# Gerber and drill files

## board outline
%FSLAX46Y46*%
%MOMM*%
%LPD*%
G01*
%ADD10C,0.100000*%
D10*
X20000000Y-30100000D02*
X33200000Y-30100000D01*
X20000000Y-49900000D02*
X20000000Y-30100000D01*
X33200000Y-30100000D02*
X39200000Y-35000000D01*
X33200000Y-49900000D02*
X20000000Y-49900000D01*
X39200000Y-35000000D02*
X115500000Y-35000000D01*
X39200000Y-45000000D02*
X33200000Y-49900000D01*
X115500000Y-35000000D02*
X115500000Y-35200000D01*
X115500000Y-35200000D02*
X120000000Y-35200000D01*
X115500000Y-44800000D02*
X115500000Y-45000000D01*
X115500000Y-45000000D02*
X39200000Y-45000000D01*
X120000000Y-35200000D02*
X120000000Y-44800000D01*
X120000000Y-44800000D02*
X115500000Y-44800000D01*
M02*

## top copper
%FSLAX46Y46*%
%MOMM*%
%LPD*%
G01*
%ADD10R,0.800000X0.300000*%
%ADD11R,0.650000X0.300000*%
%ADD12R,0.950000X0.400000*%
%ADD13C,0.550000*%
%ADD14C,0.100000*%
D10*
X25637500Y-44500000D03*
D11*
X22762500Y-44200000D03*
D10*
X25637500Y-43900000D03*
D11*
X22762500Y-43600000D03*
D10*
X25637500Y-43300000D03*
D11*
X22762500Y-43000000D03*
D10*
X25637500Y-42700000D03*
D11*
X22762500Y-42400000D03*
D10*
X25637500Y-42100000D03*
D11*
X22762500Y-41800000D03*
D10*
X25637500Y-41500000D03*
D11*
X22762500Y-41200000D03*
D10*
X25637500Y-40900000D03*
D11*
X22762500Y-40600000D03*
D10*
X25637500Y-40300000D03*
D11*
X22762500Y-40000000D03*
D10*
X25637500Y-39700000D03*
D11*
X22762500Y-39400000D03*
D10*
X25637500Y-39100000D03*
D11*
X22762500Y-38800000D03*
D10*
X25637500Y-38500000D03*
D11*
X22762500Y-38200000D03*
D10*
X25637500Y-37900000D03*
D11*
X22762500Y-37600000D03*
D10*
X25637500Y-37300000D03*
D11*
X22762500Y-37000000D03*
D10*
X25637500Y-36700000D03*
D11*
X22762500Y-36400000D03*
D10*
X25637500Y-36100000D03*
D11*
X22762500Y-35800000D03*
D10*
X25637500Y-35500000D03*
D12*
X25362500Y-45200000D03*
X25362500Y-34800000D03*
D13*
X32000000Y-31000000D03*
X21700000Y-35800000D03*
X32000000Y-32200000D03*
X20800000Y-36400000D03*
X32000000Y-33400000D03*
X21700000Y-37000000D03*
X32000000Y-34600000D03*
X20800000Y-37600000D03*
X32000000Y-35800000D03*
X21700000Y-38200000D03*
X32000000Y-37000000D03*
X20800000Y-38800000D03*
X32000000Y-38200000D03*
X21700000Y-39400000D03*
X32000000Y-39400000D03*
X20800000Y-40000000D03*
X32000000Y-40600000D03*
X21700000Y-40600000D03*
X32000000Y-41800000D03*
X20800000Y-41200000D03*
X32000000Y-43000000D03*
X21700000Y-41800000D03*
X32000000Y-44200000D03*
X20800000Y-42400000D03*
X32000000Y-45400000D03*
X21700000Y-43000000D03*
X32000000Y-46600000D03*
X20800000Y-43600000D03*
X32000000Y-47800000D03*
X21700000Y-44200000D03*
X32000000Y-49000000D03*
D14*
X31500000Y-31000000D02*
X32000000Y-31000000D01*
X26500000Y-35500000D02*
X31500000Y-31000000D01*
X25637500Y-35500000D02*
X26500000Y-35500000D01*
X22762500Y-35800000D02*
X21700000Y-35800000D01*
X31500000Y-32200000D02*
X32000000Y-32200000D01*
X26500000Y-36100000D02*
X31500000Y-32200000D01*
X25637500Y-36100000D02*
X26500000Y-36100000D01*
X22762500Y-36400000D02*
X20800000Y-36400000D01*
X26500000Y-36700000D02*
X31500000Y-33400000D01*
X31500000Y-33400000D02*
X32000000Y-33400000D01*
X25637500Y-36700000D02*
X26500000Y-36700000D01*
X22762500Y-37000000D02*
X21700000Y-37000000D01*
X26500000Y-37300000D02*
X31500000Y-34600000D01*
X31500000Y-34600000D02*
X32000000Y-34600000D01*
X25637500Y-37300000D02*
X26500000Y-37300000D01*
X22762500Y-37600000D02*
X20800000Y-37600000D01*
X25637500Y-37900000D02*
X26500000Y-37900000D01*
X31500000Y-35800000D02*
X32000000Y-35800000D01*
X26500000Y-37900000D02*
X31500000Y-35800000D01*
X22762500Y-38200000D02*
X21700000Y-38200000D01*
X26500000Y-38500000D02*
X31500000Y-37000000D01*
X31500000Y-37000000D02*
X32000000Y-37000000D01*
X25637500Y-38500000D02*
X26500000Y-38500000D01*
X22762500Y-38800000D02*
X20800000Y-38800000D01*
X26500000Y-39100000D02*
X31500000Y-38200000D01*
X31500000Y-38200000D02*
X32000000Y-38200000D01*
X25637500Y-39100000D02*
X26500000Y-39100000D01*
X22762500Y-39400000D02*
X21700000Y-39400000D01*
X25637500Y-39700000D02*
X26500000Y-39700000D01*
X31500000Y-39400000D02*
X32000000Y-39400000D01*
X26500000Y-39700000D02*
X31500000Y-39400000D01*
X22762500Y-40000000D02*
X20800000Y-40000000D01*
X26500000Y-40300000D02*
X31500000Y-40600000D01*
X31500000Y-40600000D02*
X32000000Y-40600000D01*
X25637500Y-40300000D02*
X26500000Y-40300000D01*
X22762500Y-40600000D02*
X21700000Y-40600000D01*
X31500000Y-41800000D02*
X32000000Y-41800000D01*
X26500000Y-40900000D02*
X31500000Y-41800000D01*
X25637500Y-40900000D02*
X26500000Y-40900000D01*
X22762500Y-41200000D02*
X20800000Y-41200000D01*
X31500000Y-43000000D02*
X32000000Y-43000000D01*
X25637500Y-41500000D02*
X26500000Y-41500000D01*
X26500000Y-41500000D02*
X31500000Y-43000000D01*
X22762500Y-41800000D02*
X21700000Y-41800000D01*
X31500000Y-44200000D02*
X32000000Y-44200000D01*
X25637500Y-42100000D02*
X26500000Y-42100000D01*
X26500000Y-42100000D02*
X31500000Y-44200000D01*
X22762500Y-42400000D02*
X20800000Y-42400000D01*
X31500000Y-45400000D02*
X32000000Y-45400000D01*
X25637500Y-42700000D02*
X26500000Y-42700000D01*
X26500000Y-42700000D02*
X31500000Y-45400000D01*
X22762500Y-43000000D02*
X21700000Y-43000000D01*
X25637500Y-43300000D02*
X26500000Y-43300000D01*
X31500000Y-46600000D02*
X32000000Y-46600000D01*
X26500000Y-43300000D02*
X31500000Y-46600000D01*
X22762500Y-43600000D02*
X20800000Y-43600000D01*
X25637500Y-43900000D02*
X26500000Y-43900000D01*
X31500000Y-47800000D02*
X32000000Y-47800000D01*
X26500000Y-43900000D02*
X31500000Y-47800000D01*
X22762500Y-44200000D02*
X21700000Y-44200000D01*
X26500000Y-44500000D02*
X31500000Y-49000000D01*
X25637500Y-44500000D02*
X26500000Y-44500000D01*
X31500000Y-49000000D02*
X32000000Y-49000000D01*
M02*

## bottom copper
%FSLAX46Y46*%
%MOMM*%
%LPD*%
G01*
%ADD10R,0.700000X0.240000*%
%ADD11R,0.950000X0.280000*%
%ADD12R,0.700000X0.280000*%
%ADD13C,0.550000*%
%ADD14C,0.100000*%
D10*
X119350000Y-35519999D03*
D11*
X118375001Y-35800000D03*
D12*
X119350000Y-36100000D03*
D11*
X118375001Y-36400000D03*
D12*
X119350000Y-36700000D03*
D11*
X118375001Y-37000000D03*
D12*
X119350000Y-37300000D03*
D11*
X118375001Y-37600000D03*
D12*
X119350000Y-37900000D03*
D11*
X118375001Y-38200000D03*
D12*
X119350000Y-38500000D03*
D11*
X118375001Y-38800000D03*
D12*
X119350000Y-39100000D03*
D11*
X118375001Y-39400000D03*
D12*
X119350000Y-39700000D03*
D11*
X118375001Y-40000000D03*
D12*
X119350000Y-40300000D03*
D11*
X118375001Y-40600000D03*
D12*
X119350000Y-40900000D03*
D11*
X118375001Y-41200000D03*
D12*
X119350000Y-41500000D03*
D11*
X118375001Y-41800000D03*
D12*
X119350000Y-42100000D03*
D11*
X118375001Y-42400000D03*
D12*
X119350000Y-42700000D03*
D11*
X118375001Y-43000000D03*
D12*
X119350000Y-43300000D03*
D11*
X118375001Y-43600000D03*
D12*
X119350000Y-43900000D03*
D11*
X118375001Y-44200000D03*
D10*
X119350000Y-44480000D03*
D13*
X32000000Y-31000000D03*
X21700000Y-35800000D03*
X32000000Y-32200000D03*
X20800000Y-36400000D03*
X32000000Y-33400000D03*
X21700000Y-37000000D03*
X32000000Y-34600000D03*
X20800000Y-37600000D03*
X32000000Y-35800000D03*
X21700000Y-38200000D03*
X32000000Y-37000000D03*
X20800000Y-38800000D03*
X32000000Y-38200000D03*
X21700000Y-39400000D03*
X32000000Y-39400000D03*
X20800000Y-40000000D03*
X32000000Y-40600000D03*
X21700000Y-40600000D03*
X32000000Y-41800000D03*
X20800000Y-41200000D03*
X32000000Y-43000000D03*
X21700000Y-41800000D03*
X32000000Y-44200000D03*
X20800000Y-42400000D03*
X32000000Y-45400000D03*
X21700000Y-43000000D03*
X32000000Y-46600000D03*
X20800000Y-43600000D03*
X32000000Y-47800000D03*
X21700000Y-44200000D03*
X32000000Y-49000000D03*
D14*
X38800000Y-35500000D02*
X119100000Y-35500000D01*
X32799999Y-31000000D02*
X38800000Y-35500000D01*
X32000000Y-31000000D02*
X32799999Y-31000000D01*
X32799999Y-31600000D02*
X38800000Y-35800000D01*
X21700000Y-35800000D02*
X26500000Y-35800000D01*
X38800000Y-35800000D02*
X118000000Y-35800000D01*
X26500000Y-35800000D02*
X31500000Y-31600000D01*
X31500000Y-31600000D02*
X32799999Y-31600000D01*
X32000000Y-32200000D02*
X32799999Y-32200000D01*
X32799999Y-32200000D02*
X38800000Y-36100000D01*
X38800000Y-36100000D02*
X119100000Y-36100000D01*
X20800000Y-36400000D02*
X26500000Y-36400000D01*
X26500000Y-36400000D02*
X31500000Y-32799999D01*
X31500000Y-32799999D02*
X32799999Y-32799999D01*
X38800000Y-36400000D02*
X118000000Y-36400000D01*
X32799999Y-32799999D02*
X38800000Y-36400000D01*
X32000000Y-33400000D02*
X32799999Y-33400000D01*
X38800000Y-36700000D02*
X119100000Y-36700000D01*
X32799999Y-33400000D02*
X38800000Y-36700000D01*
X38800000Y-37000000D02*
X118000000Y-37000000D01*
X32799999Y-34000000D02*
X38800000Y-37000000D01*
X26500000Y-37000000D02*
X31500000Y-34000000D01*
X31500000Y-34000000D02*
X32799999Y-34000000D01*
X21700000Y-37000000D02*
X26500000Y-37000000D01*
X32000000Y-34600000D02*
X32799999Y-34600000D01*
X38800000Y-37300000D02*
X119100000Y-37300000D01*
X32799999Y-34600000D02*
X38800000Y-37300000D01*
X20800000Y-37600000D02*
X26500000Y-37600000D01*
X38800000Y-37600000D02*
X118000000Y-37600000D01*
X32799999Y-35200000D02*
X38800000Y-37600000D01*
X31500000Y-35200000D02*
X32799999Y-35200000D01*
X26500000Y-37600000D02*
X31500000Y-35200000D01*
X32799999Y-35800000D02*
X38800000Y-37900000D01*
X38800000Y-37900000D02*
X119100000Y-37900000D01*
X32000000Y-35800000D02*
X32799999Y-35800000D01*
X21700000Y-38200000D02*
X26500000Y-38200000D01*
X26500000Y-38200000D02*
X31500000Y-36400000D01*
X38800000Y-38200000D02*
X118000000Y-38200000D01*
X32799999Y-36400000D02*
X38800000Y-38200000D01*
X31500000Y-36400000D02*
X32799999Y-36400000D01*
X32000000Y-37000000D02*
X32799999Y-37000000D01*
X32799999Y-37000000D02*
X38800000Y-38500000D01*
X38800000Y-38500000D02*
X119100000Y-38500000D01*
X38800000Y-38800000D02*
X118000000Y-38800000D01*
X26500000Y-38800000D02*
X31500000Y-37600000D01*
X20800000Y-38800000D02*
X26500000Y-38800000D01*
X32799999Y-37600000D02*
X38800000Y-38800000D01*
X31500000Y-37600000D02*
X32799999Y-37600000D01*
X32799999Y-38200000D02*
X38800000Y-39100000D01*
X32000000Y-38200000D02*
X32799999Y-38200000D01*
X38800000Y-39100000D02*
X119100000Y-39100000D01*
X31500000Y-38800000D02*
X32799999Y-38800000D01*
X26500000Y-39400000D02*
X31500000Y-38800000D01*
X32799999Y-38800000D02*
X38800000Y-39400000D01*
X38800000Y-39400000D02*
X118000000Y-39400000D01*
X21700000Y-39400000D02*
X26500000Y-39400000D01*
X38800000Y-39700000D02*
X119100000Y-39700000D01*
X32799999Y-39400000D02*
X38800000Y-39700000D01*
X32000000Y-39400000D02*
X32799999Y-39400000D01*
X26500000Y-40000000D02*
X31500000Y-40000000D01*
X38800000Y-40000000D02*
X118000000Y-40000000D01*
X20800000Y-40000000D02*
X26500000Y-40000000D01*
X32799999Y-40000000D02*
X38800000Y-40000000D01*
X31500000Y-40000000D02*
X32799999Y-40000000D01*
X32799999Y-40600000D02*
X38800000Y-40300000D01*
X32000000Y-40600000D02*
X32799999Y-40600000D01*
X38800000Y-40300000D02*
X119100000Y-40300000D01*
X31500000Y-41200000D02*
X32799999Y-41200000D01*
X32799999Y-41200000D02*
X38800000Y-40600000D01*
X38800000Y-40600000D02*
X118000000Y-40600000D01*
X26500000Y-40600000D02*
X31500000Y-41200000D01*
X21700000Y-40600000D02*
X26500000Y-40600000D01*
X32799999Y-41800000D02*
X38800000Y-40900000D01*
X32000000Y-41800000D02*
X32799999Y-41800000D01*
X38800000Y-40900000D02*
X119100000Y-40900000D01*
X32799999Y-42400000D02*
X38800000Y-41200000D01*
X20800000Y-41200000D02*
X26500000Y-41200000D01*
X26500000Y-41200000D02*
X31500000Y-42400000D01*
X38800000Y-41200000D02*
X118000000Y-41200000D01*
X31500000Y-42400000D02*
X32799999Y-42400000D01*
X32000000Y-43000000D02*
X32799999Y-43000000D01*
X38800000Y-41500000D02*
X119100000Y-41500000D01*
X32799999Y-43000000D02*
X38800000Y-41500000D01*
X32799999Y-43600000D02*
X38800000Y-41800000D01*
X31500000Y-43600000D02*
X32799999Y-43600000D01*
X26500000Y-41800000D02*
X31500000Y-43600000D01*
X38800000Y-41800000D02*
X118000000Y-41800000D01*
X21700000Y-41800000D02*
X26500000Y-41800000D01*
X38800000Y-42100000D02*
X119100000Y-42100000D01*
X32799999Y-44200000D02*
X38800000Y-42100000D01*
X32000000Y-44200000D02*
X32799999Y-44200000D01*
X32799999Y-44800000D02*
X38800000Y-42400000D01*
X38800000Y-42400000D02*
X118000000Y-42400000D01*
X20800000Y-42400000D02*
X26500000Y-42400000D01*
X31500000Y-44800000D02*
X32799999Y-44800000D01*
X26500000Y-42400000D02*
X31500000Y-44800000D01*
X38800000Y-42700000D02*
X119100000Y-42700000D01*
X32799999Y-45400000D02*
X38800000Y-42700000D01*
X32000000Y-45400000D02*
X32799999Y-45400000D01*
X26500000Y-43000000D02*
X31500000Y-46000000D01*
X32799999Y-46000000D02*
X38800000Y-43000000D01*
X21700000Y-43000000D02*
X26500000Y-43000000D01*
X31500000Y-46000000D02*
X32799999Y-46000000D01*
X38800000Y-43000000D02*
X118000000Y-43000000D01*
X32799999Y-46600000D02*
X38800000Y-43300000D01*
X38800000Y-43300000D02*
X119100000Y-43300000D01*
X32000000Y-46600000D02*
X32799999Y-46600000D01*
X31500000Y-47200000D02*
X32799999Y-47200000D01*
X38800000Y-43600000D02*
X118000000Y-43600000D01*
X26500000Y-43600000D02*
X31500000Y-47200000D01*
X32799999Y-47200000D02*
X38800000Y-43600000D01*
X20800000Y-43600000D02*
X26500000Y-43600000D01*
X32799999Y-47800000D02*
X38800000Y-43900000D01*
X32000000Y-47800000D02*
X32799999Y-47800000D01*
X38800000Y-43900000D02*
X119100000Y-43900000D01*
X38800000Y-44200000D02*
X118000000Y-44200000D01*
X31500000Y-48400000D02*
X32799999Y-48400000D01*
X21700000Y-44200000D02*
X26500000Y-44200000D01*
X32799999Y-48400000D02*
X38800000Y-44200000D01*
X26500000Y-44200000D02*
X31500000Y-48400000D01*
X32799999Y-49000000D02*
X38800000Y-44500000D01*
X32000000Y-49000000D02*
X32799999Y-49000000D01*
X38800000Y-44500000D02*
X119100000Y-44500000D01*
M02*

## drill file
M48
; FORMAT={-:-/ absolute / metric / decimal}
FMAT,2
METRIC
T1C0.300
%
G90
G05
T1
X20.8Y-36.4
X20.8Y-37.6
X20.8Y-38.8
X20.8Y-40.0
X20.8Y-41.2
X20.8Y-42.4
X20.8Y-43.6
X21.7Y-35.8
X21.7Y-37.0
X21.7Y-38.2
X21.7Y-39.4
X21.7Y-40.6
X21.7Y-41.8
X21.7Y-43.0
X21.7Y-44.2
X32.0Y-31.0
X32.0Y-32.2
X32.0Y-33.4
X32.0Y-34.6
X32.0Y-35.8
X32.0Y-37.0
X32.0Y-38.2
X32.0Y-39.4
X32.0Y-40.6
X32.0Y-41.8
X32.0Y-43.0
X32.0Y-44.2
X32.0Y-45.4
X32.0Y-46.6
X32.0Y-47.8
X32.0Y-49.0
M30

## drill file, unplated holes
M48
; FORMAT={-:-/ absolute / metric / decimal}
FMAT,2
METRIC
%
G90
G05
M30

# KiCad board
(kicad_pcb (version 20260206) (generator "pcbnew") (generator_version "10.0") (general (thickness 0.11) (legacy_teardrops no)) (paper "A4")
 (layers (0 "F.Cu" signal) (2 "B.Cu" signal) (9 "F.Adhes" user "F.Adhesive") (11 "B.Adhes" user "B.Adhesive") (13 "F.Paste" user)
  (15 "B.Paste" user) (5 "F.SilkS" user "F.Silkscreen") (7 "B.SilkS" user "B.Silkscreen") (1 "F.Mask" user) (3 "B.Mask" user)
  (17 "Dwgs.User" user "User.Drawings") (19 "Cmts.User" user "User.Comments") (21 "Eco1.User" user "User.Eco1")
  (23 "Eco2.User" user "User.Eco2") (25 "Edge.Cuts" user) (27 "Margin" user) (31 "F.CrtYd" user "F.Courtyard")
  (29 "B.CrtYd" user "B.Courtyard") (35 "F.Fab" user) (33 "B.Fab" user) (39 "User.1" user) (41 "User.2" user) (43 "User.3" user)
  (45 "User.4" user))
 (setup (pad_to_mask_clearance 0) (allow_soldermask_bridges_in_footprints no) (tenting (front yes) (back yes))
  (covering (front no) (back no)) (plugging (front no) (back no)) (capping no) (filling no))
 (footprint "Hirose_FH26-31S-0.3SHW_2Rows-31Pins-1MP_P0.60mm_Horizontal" (layer "F.Cu") (at 24.2375 40 180)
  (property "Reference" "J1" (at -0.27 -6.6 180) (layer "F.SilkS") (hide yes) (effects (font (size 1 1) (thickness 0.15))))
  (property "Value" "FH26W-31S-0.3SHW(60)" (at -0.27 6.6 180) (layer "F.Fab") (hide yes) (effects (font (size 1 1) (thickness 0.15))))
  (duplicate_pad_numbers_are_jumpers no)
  (pad "1" smd rect (at -1.4 -4.5 180) (size 0.8 0.3) (layers "F.Cu" "F.Mask" "F.Paste") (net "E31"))
  (pad "2" smd rect (at 1.475 -4.2 180) (size 0.65 0.3) (layers "F.Cu" "F.Mask" "F.Paste") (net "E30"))
  (pad "3" smd rect (at -1.4 -3.9 180) (size 0.8 0.3) (layers "F.Cu" "F.Mask" "F.Paste") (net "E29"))
  (pad "4" smd rect (at 1.475 -3.6 180) (size 0.65 0.3) (layers "F.Cu" "F.Mask" "F.Paste") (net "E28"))
  (pad "5" smd rect (at -1.4 -3.3 180) (size 0.8 0.3) (layers "F.Cu" "F.Mask" "F.Paste") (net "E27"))
  (pad "6" smd rect (at 1.475 -3 180) (size 0.65 0.3) (layers "F.Cu" "F.Mask" "F.Paste") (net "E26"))
  (pad "7" smd rect (at -1.4 -2.7 180) (size 0.8 0.3) (layers "F.Cu" "F.Mask" "F.Paste") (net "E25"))
  (pad "8" smd rect (at 1.475 -2.4 180) (size 0.65 0.3) (layers "F.Cu" "F.Mask" "F.Paste") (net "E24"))
  (pad "9" smd rect (at -1.4 -2.1 180) (size 0.8 0.3) (layers "F.Cu" "F.Mask" "F.Paste") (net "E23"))
  (pad "10" smd rect (at 1.475 -1.8 180) (size 0.65 0.3) (layers "F.Cu" "F.Mask" "F.Paste") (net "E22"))
  (pad "11" smd rect (at -1.4 -1.5 180) (size 0.8 0.3) (layers "F.Cu" "F.Mask" "F.Paste") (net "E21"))
  (pad "12" smd rect (at 1.475 -1.2 180) (size 0.65 0.3) (layers "F.Cu" "F.Mask" "F.Paste") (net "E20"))
  (pad "13" smd rect (at -1.4 -0.9 180) (size 0.8 0.3) (layers "F.Cu" "F.Mask" "F.Paste") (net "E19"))
  (pad "14" smd rect (at 1.475 -0.6 180) (size 0.65 0.3) (layers "F.Cu" "F.Mask" "F.Paste") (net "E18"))
  (pad "15" smd rect (at -1.4 -0.3 180) (size 0.8 0.3) (layers "F.Cu" "F.Mask" "F.Paste") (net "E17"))
  (pad "16" smd rect (at 1.475 0 180) (size 0.65 0.3) (layers "F.Cu" "F.Mask" "F.Paste") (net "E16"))
  (pad "17" smd rect (at -1.4 0.3 180) (size 0.8 0.3) (layers "F.Cu" "F.Mask" "F.Paste") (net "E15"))
  (pad "18" smd rect (at 1.475 0.6 180) (size 0.65 0.3) (layers "F.Cu" "F.Mask" "F.Paste") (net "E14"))
  (pad "19" smd rect (at -1.4 0.9 180) (size 0.8 0.3) (layers "F.Cu" "F.Mask" "F.Paste") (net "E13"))
  (pad "20" smd rect (at 1.475 1.2 180) (size 0.65 0.3) (layers "F.Cu" "F.Mask" "F.Paste") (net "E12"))
  (pad "21" smd rect (at -1.4 1.5 180) (size 0.8 0.3) (layers "F.Cu" "F.Mask" "F.Paste") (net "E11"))
  (pad "22" smd rect (at 1.475 1.8 180) (size 0.65 0.3) (layers "F.Cu" "F.Mask" "F.Paste") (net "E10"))
  (pad "23" smd rect (at -1.4 2.1 180) (size 0.8 0.3) (layers "F.Cu" "F.Mask" "F.Paste") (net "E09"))
  (pad "24" smd rect (at 1.475 2.4 180) (size 0.65 0.3) (layers "F.Cu" "F.Mask" "F.Paste") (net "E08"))
  (pad "25" smd rect (at -1.4 2.7 180) (size 0.8 0.3) (layers "F.Cu" "F.Mask" "F.Paste") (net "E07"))
  (pad "26" smd rect (at 1.475 3 180) (size 0.65 0.3) (layers "F.Cu" "F.Mask" "F.Paste") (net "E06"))
  (pad "27" smd rect (at -1.4 3.3 180) (size 0.8 0.3) (layers "F.Cu" "F.Mask" "F.Paste") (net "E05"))
  (pad "28" smd rect (at 1.475 3.6 180) (size 0.65 0.3) (layers "F.Cu" "F.Mask" "F.Paste") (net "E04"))
  (pad "29" smd rect (at -1.4 3.9 180) (size 0.8 0.3) (layers "F.Cu" "F.Mask" "F.Paste") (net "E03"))
  (pad "30" smd rect (at 1.475 4.2 180) (size 0.65 0.3) (layers "F.Cu" "F.Mask" "F.Paste") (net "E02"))
  (pad "31" smd rect (at -1.4 4.5 180) (size 0.8 0.3) (layers "F.Cu" "F.Mask" "F.Paste") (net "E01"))
  (pad "MP" smd rect (at -1.125 -5.2 180) (size 0.95 0.4) (layers "F.Cu" "F.Mask" "F.Paste"))
  (pad "MP" smd rect (at -1.125 5.2 180) (size 0.95 0.4) (layers "F.Cu" "F.Mask" "F.Paste")))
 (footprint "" (layer "B.Cu") (at 118.6 40 180)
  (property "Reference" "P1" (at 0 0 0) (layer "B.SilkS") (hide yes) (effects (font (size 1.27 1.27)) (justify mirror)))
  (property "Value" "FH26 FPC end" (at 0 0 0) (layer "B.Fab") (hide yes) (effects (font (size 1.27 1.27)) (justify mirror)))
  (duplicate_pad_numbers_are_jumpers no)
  (pad "1" smd rect (at -0.75 4.480001 180) (size 0.7 0.24) (layers "B.Cu" "B.Mask") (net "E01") (thermal_bridge_angle 45))
  (pad "2" smd rect (at 0.224999 4.2 180) (size 0.95 0.28) (layers "B.Cu" "B.Mask") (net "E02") (thermal_bridge_angle 45))
  (pad "3" smd rect (at -0.75 3.9 180) (size 0.7 0.28) (layers "B.Cu" "B.Mask") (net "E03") (thermal_bridge_angle 45))
  (pad "4" smd rect (at 0.224999 3.6 180) (size 0.95 0.28) (layers "B.Cu" "B.Mask") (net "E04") (thermal_bridge_angle 45))
  (pad "5" smd rect (at -0.75 3.3 180) (size 0.7 0.28) (layers "B.Cu" "B.Mask") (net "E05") (thermal_bridge_angle 45))
  (pad "6" smd rect (at 0.224999 3 180) (size 0.95 0.28) (layers "B.Cu" "B.Mask") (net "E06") (thermal_bridge_angle 45))
  (pad "7" smd rect (at -0.75 2.7 180) (size 0.7 0.28) (layers "B.Cu" "B.Mask") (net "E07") (thermal_bridge_angle 45))
  (pad "8" smd rect (at 0.224999 2.4 180) (size 0.95 0.28) (layers "B.Cu" "B.Mask") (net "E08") (thermal_bridge_angle 45))
  (pad "9" smd rect (at -0.75 2.1 180) (size 0.7 0.28) (layers "B.Cu" "B.Mask") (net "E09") (thermal_bridge_angle 45))
  (pad "10" smd rect (at 0.224999 1.8 180) (size 0.95 0.28) (layers "B.Cu" "B.Mask") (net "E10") (thermal_bridge_angle 45))
  (pad "11" smd rect (at -0.75 1.5 180) (size 0.7 0.28) (layers "B.Cu" "B.Mask") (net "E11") (thermal_bridge_angle 45))
  (pad "12" smd rect (at 0.224999 1.2 180) (size 0.95 0.28) (layers "B.Cu" "B.Mask") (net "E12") (thermal_bridge_angle 45))
  (pad "13" smd rect (at -0.75 0.9 180) (size 0.7 0.28) (layers "B.Cu" "B.Mask") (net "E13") (thermal_bridge_angle 45))
  (pad "14" smd rect (at 0.224999 0.6 180) (size 0.95 0.28) (layers "B.Cu" "B.Mask") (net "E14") (thermal_bridge_angle 45))
  (pad "15" smd rect (at -0.75 0.3 180) (size 0.7 0.28) (layers "B.Cu" "B.Mask") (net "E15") (thermal_bridge_angle 45))
  (pad "16" smd rect (at 0.224999 0 180) (size 0.95 0.28) (layers "B.Cu" "B.Mask") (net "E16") (thermal_bridge_angle 45))
  (pad "17" smd rect (at -0.75 -0.3 180) (size 0.7 0.28) (layers "B.Cu" "B.Mask") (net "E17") (thermal_bridge_angle 45))
  (pad "18" smd rect (at 0.224999 -0.6 180) (size 0.95 0.28) (layers "B.Cu" "B.Mask") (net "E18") (thermal_bridge_angle 45))
  (pad "19" smd rect (at -0.75 -0.9 180) (size 0.7 0.28) (layers "B.Cu" "B.Mask") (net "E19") (thermal_bridge_angle 45))
  (pad "20" smd rect (at 0.224999 -1.2 180) (size 0.95 0.28) (layers "B.Cu" "B.Mask") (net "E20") (thermal_bridge_angle 45))
  (pad "21" smd rect (at -0.75 -1.5 180) (size 0.7 0.28) (layers "B.Cu" "B.Mask") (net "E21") (thermal_bridge_angle 45))
  (pad "22" smd rect (at 0.224999 -1.8 180) (size 0.95 0.28) (layers "B.Cu" "B.Mask") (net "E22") (thermal_bridge_angle 45))
  (pad "23" smd rect (at -0.75 -2.1 180) (size 0.7 0.28) (layers "B.Cu" "B.Mask") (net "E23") (thermal_bridge_angle 45))
  (pad "24" smd rect (at 0.224999 -2.4 180) (size 0.95 0.28) (layers "B.Cu" "B.Mask") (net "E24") (thermal_bridge_angle 45))
  (pad "25" smd rect (at -0.75 -2.7 180) (size 0.7 0.28) (layers "B.Cu" "B.Mask") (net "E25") (thermal_bridge_angle 45))
  (pad "26" smd rect (at 0.224999 -3 180) (size 0.95 0.28) (layers "B.Cu" "B.Mask") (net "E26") (thermal_bridge_angle 45))
  (pad "27" smd rect (at -0.75 -3.3 180) (size 0.7 0.28) (layers "B.Cu" "B.Mask") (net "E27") (thermal_bridge_angle 45))
  (pad "28" smd rect (at 0.224999 -3.6 180) (size 0.95 0.28) (layers "B.Cu" "B.Mask") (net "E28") (thermal_bridge_angle 45))
  (pad "29" smd rect (at -0.75 -3.9 180) (size 0.7 0.28) (layers "B.Cu" "B.Mask") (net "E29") (thermal_bridge_angle 45))
  (pad "30" smd rect (at 0.224999 -4.2 180) (size 0.95 0.28) (layers "B.Cu" "B.Mask") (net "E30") (thermal_bridge_angle 45))
  (pad "31" smd rect (at -0.75 -4.48 180) (size 0.7 0.24) (layers "B.Cu" "B.Mask") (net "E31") (thermal_bridge_angle 45)))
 (gr_line (start 20 30.1) (end 33.2 30.1) (stroke (width 0.1) (type default)) (layer "Edge.Cuts"))
 (gr_line (start 20 49.9) (end 20 30.1) (stroke (width 0.1) (type default)) (layer "Edge.Cuts"))
 (gr_line (start 33.2 30.1) (end 39.2 35) (stroke (width 0.1) (type default)) (layer "Edge.Cuts"))
 (gr_line (start 33.2 49.9) (end 20 49.9) (stroke (width 0.1) (type default)) (layer "Edge.Cuts"))
 (gr_line (start 39.2 35) (end 115.5 35) (stroke (width 0.1) (type default)) (layer "Edge.Cuts"))
 (gr_line (start 39.2 45) (end 33.2 49.9) (stroke (width 0.1) (type default)) (layer "Edge.Cuts"))
 (gr_line (start 115.5 35) (end 115.5 35.2) (stroke (width 0.1) (type default)) (layer "Edge.Cuts"))
 (gr_line (start 115.5 35.2) (end 120 35.2) (stroke (width 0.1) (type default)) (layer "Edge.Cuts"))
 (gr_line (start 115.5 44.8) (end 115.5 45) (stroke (width 0.1) (type default)) (layer "Edge.Cuts"))
 (gr_line (start 115.5 45) (end 39.2 45) (stroke (width 0.1) (type default)) (layer "Edge.Cuts"))
 (gr_line (start 120 35.2) (end 120 44.8) (stroke (width 0.1) (type default)) (layer "Edge.Cuts"))
 (gr_line (start 120 44.8) (end 115.5 44.8) (stroke (width 0.1) (type default)) (layer "Edge.Cuts"))
 (segment (start 31.5 31) (end 32 31) (width 0.1) (layer "F.Cu") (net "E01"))
 (segment (start 26.5 35.5) (end 31.5 31) (width 0.1) (layer "F.Cu") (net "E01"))
 (segment (start 25.6375 35.5) (end 26.5 35.5) (width 0.1) (layer "F.Cu") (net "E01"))
 (via (at 32 31) (size 0.55) (drill 0.3) (layers "F.Cu" "B.Cu") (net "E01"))
 (segment (start 38.8 35.5) (end 119.1 35.5) (width 0.1) (layer "B.Cu") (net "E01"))
 (segment (start 32.799999 31) (end 38.8 35.5) (width 0.1) (layer "B.Cu") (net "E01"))
 (segment (start 32 31) (end 32.799999 31) (width 0.1) (layer "B.Cu") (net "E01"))
 (segment (start 22.7625 35.8) (end 21.7 35.8) (width 0.1) (layer "F.Cu") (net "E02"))
 (via (at 21.7 35.8) (size 0.55) (drill 0.3) (layers "F.Cu" "B.Cu") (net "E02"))
 (segment (start 32.799999 31.6) (end 38.8 35.8) (width 0.1) (layer "B.Cu") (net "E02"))
 (segment (start 21.7 35.8) (end 26.5 35.8) (width 0.1) (layer "B.Cu") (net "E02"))
 (segment (start 38.8 35.8) (end 118 35.8) (width 0.1) (layer "B.Cu") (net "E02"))
 (segment (start 26.5 35.8) (end 31.5 31.6) (width 0.1) (layer "B.Cu") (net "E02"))
 (segment (start 31.5 31.6) (end 32.799999 31.6) (width 0.1) (layer "B.Cu") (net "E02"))
 (segment (start 31.5 32.2) (end 32 32.2) (width 0.1) (layer "F.Cu") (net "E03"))
 (segment (start 26.5 36.1) (end 31.5 32.2) (width 0.1) (layer "F.Cu") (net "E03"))
 (segment (start 25.6375 36.1) (end 26.5 36.1) (width 0.1) (layer "F.Cu") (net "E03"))
 (via (at 32 32.2) (size 0.55) (drill 0.3) (layers "F.Cu" "B.Cu") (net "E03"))
 (segment (start 32 32.2) (end 32.799999 32.2) (width 0.1) (layer "B.Cu") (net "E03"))
 (segment (start 32.799999 32.2) (end 38.8 36.1) (width 0.1) (layer "B.Cu") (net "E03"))
 (segment (start 38.8 36.1) (end 119.1 36.1) (width 0.1) (layer "B.Cu") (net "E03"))
 (segment (start 22.7625 36.4) (end 20.8 36.4) (width 0.1) (layer "F.Cu") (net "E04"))
 (via (at 20.8 36.4) (size 0.55) (drill 0.3) (layers "F.Cu" "B.Cu") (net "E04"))
 (segment (start 20.8 36.4) (end 26.5 36.4) (width 0.1) (layer "B.Cu") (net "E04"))
 (segment (start 26.5 36.4) (end 31.5 32.799999) (width 0.1) (layer "B.Cu") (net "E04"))
 (segment (start 31.5 32.799999) (end 32.799999 32.799999) (width 0.1) (layer "B.Cu") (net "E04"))
 (segment (start 38.8 36.4) (end 118 36.4) (width 0.1) (layer "B.Cu") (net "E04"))
 (segment (start 32.799999 32.799999) (end 38.8 36.4) (width 0.1) (layer "B.Cu") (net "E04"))
 (segment (start 26.5 36.7) (end 31.5 33.4) (width 0.1) (layer "F.Cu") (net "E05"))
 (segment (start 31.5 33.4) (end 32 33.4) (width 0.1) (layer "F.Cu") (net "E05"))
 (segment (start 25.6375 36.7) (end 26.5 36.7) (width 0.1) (layer "F.Cu") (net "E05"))
 (via (at 32 33.4) (size 0.55) (drill 0.3) (layers "F.Cu" "B.Cu") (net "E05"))
 (segment (start 32 33.4) (end 32.799999 33.4) (width 0.1) (layer "B.Cu") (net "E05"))
 (segment (start 38.8 36.7) (end 119.1 36.7) (width 0.1) (layer "B.Cu") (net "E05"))
 (segment (start 32.799999 33.4) (end 38.8 36.7) (width 0.1) (layer "B.Cu") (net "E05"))
 (segment (start 22.7625 37) (end 21.7 37) (width 0.1) (layer "F.Cu") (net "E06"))
 (via (at 21.7 37) (size 0.55) (drill 0.3) (layers "F.Cu" "B.Cu") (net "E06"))
 (segment (start 38.8 37) (end 118 37) (width 0.1) (layer "B.Cu") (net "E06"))
 (segment (start 32.799999 34) (end 38.8 37) (width 0.1) (layer "B.Cu") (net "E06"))
 (segment (start 26.5 37) (end 31.5 34) (width 0.1) (layer "B.Cu") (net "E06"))
 (segment (start 31.5 34) (end 32.799999 34) (width 0.1) (layer "B.Cu") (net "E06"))
 (segment (start 21.7 37) (end 26.5 37) (width 0.1) (layer "B.Cu") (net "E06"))
 (segment (start 26.5 37.3) (end 31.5 34.6) (width 0.1) (layer "F.Cu") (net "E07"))
 (segment (start 31.5 34.6) (end 32 34.6) (width 0.1) (layer "F.Cu") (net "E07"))
 (segment (start 25.6375 37.3) (end 26.5 37.3) (width 0.1) (layer "F.Cu") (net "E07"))
 (via (at 32 34.6) (size 0.55) (drill 0.3) (layers "F.Cu" "B.Cu") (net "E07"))
 (segment (start 32 34.6) (end 32.799999 34.6) (width 0.1) (layer "B.Cu") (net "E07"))
 (segment (start 38.8 37.3) (end 119.1 37.3) (width 0.1) (layer "B.Cu") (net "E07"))
 (segment (start 32.799999 34.6) (end 38.8 37.3) (width 0.1) (layer "B.Cu") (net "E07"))
 (segment (start 22.7625 37.6) (end 20.8 37.6) (width 0.1) (layer "F.Cu") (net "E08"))
 (via (at 20.8 37.6) (size 0.55) (drill 0.3) (layers "F.Cu" "B.Cu") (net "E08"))
 (segment (start 20.8 37.6) (end 26.5 37.6) (width 0.1) (layer "B.Cu") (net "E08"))
 (segment (start 38.8 37.6) (end 118 37.6) (width 0.1) (layer "B.Cu") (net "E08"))
 (segment (start 32.799999 35.2) (end 38.8 37.6) (width 0.1) (layer "B.Cu") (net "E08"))
 (segment (start 31.5 35.2) (end 32.799999 35.2) (width 0.1) (layer "B.Cu") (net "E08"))
 (segment (start 26.5 37.6) (end 31.5 35.2) (width 0.1) (layer "B.Cu") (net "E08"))
 (segment (start 25.6375 37.9) (end 26.5 37.9) (width 0.1) (layer "F.Cu") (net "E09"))
 (segment (start 31.5 35.8) (end 32 35.8) (width 0.1) (layer "F.Cu") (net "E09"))
 (segment (start 26.5 37.9) (end 31.5 35.8) (width 0.1) (layer "F.Cu") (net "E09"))
 (via (at 32 35.8) (size 0.55) (drill 0.3) (layers "F.Cu" "B.Cu") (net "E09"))
 (segment (start 32.799999 35.8) (end 38.8 37.9) (width 0.1) (layer "B.Cu") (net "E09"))
 (segment (start 38.8 37.9) (end 119.1 37.9) (width 0.1) (layer "B.Cu") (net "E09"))
 (segment (start 32 35.8) (end 32.799999 35.8) (width 0.1) (layer "B.Cu") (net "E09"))
 (segment (start 22.7625 38.2) (end 21.7 38.2) (width 0.1) (layer "F.Cu") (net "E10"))
 (via (at 21.7 38.2) (size 0.55) (drill 0.3) (layers "F.Cu" "B.Cu") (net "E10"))
 (segment (start 21.7 38.2) (end 26.5 38.2) (width 0.1) (layer "B.Cu") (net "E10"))
 (segment (start 26.5 38.2) (end 31.5 36.4) (width 0.1) (layer "B.Cu") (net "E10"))
 (segment (start 38.8 38.2) (end 118 38.2) (width 0.1) (layer "B.Cu") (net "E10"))
 (segment (start 32.799999 36.4) (end 38.8 38.2) (width 0.1) (layer "B.Cu") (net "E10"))
 (segment (start 31.5 36.4) (end 32.799999 36.4) (width 0.1) (layer "B.Cu") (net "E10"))
 (segment (start 26.5 38.5) (end 31.5 37) (width 0.1) (layer "F.Cu") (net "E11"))
 (segment (start 31.5 37) (end 32 37) (width 0.1) (layer "F.Cu") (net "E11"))
 (segment (start 25.6375 38.5) (end 26.5 38.5) (width 0.1) (layer "F.Cu") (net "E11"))
 (via (at 32 37) (size 0.55) (drill 0.3) (layers "F.Cu" "B.Cu") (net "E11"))
 (segment (start 32 37) (end 32.799999 37) (width 0.1) (layer "B.Cu") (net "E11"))
 (segment (start 32.799999 37) (end 38.8 38.5) (width 0.1) (layer "B.Cu") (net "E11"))
 (segment (start 38.8 38.5) (end 119.1 38.5) (width 0.1) (layer "B.Cu") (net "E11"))
 (segment (start 22.7625 38.8) (end 20.8 38.8) (width 0.1) (layer "F.Cu") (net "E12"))
 (via (at 20.8 38.8) (size 0.55) (drill 0.3) (layers "F.Cu" "B.Cu") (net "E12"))
 (segment (start 38.8 38.8) (end 118 38.8) (width 0.1) (layer "B.Cu") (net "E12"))
 (segment (start 26.5 38.8) (end 31.5 37.6) (width 0.1) (layer "B.Cu") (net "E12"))
 (segment (start 20.8 38.8) (end 26.5 38.8) (width 0.1) (layer "B.Cu") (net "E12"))
 (segment (start 32.799999 37.6) (end 38.8 38.8) (width 0.1) (layer "B.Cu") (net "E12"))
 (segment (start 31.5 37.6) (end 32.799999 37.6) (width 0.1) (layer "B.Cu") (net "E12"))
 (segment (start 26.5 39.1) (end 31.5 38.2) (width 0.1) (layer "F.Cu") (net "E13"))
 (segment (start 31.5 38.2) (end 32 38.2) (width 0.1) (layer "F.Cu") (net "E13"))
 (segment (start 25.6375 39.1) (end 26.5 39.1) (width 0.1) (layer "F.Cu") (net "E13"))
 (via (at 32 38.2) (size 0.55) (drill 0.3) (layers "F.Cu" "B.Cu") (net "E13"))
 (segment (start 32.799999 38.2) (end 38.8 39.1) (width 0.1) (layer "B.Cu") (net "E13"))
 (segment (start 32 38.2) (end 32.799999 38.2) (width 0.1) (layer "B.Cu") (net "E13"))
 (segment (start 38.8 39.1) (end 119.1 39.1) (width 0.1) (layer "B.Cu") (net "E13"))
 (segment (start 22.7625 39.4) (end 21.7 39.4) (width 0.1) (layer "F.Cu") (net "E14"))
 (via (at 21.7 39.4) (size 0.55) (drill 0.3) (layers "F.Cu" "B.Cu") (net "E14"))
 (segment (start 31.5 38.8) (end 32.799999 38.8) (width 0.1) (layer "B.Cu") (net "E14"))
 (segment (start 26.5 39.4) (end 31.5 38.8) (width 0.1) (layer "B.Cu") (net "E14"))
 (segment (start 32.799999 38.8) (end 38.8 39.4) (width 0.1) (layer "B.Cu") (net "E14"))
 (segment (start 38.8 39.4) (end 118 39.4) (width 0.1) (layer "B.Cu") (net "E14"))
 (segment (start 21.7 39.4) (end 26.5 39.4) (width 0.1) (layer "B.Cu") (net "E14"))
 (segment (start 25.6375 39.7) (end 26.5 39.7) (width 0.1) (layer "F.Cu") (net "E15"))
 (segment (start 31.5 39.4) (end 32 39.4) (width 0.1) (layer "F.Cu") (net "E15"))
 (segment (start 26.5 39.7) (end 31.5 39.4) (width 0.1) (layer "F.Cu") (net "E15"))
 (via (at 32 39.4) (size 0.55) (drill 0.3) (layers "F.Cu" "B.Cu") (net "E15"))
 (segment (start 38.8 39.7) (end 119.1 39.7) (width 0.1) (layer "B.Cu") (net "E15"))
 (segment (start 32.799999 39.4) (end 38.8 39.7) (width 0.1) (layer "B.Cu") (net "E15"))
 (segment (start 32 39.4) (end 32.799999 39.4) (width 0.1) (layer "B.Cu") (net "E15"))
 (segment (start 22.7625 40) (end 20.8 40) (width 0.1) (layer "F.Cu") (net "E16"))
 (via (at 20.8 40) (size 0.55) (drill 0.3) (layers "F.Cu" "B.Cu") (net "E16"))
 (segment (start 26.5 40) (end 31.5 40) (width 0.1) (layer "B.Cu") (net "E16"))
 (segment (start 38.8 40) (end 118 40) (width 0.1) (layer "B.Cu") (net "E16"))
 (segment (start 20.8 40) (end 26.5 40) (width 0.1) (layer "B.Cu") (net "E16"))
 (segment (start 32.799999 40) (end 38.8 40) (width 0.1) (layer "B.Cu") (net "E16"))
 (segment (start 31.5 40) (end 32.799999 40) (width 0.1) (layer "B.Cu") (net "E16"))
 (segment (start 26.5 40.3) (end 31.5 40.6) (width 0.1) (layer "F.Cu") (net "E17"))
 (segment (start 31.5 40.6) (end 32 40.6) (width 0.1) (layer "F.Cu") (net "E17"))
 (segment (start 25.6375 40.3) (end 26.5 40.3) (width 0.1) (layer "F.Cu") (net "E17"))
 (via (at 32 40.6) (size 0.55) (drill 0.3) (layers "F.Cu" "B.Cu") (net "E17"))
 (segment (start 32.799999 40.6) (end 38.8 40.3) (width 0.1) (layer "B.Cu") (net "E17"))
 (segment (start 32 40.6) (end 32.799999 40.6) (width 0.1) (layer "B.Cu") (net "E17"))
 (segment (start 38.8 40.3) (end 119.1 40.3) (width 0.1) (layer "B.Cu") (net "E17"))
 (segment (start 22.7625 40.6) (end 21.7 40.6) (width 0.1) (layer "F.Cu") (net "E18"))
 (via (at 21.7 40.6) (size 0.55) (drill 0.3) (layers "F.Cu" "B.Cu") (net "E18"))
 (segment (start 31.5 41.2) (end 32.799999 41.2) (width 0.1) (layer "B.Cu") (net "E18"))
 (segment (start 32.799999 41.2) (end 38.8 40.6) (width 0.1) (layer "B.Cu") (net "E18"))
 (segment (start 38.8 40.6) (end 118 40.6) (width 0.1) (layer "B.Cu") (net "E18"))
 (segment (start 26.5 40.6) (end 31.5 41.2) (width 0.1) (layer "B.Cu") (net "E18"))
 (segment (start 21.7 40.6) (end 26.5 40.6) (width 0.1) (layer "B.Cu") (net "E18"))
 (segment (start 31.5 41.8) (end 32 41.8) (width 0.1) (layer "F.Cu") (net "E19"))
 (segment (start 26.5 40.9) (end 31.5 41.8) (width 0.1) (layer "F.Cu") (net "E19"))
 (segment (start 25.6375 40.9) (end 26.5 40.9) (width 0.1) (layer "F.Cu") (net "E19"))
 (via (at 32 41.8) (size 0.55) (drill 0.3) (layers "F.Cu" "B.Cu") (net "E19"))
 (segment (start 32.799999 41.8) (end 38.8 40.9) (width 0.1) (layer "B.Cu") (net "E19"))
 (segment (start 32 41.8) (end 32.799999 41.8) (width 0.1) (layer "B.Cu") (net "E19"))
 (segment (start 38.8 40.9) (end 119.1 40.9) (width 0.1) (layer "B.Cu") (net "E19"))
 (segment (start 22.7625 41.2) (end 20.8 41.2) (width 0.1) (layer "F.Cu") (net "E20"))
 (via (at 20.8 41.2) (size 0.55) (drill 0.3) (layers "F.Cu" "B.Cu") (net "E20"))
 (segment (start 32.799999 42.4) (end 38.8 41.2) (width 0.1) (layer "B.Cu") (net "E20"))
 (segment (start 20.8 41.2) (end 26.5 41.2) (width 0.1) (layer "B.Cu") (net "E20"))
 (segment (start 26.5 41.2) (end 31.5 42.4) (width 0.1) (layer "B.Cu") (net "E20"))
 (segment (start 38.8 41.2) (end 118 41.2) (width 0.1) (layer "B.Cu") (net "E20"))
 (segment (start 31.5 42.4) (end 32.799999 42.4) (width 0.1) (layer "B.Cu") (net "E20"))
 (segment (start 31.5 43) (end 32 43) (width 0.1) (layer "F.Cu") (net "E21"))
 (segment (start 25.6375 41.5) (end 26.5 41.5) (width 0.1) (layer "F.Cu") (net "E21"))
 (segment (start 26.5 41.5) (end 31.5 43) (width 0.1) (layer "F.Cu") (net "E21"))
 (via (at 32 43) (size 0.55) (drill 0.3) (layers "F.Cu" "B.Cu") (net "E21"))
 (segment (start 32 43) (end 32.799999 43) (width 0.1) (layer "B.Cu") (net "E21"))
 (segment (start 38.8 41.5) (end 119.1 41.5) (width 0.1) (layer "B.Cu") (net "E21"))
 (segment (start 32.799999 43) (end 38.8 41.5) (width 0.1) (layer "B.Cu") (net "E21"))
 (segment (start 22.7625 41.8) (end 21.7 41.8) (width 0.1) (layer "F.Cu") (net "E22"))
 (via (at 21.7 41.8) (size 0.55) (drill 0.3) (layers "F.Cu" "B.Cu") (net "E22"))
 (segment (start 32.799999 43.6) (end 38.8 41.8) (width 0.1) (layer "B.Cu") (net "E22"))
 (segment (start 31.5 43.6) (end 32.799999 43.6) (width 0.1) (layer "B.Cu") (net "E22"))
 (segment (start 26.5 41.8) (end 31.5 43.6) (width 0.1) (layer "B.Cu") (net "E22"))
 (segment (start 38.8 41.8) (end 118 41.8) (width 0.1) (layer "B.Cu") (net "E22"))
 (segment (start 21.7 41.8) (end 26.5 41.8) (width 0.1) (layer "B.Cu") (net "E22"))
 (segment (start 31.5 44.2) (end 32 44.2) (width 0.1) (layer "F.Cu") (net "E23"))
 (segment (start 25.6375 42.1) (end 26.5 42.1) (width 0.1) (layer "F.Cu") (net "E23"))
 (segment (start 26.5 42.1) (end 31.5 44.2) (width 0.1) (layer "F.Cu") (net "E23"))
 (via (at 32 44.2) (size 0.55) (drill 0.3) (layers "F.Cu" "B.Cu") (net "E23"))
 (segment (start 38.8 42.1) (end 119.1 42.1) (width 0.1) (layer "B.Cu") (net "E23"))
 (segment (start 32.799999 44.2) (end 38.8 42.1) (width 0.1) (layer "B.Cu") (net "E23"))
 (segment (start 32 44.2) (end 32.799999 44.2) (width 0.1) (layer "B.Cu") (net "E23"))
 (segment (start 22.7625 42.4) (end 20.8 42.4) (width 0.1) (layer "F.Cu") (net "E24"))
 (via (at 20.8 42.4) (size 0.55) (drill 0.3) (layers "F.Cu" "B.Cu") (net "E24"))
 (segment (start 32.799999 44.8) (end 38.8 42.4) (width 0.1) (layer "B.Cu") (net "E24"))
 (segment (start 38.8 42.4) (end 118 42.4) (width 0.1) (layer "B.Cu") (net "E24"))
 (segment (start 20.8 42.4) (end 26.5 42.4) (width 0.1) (layer "B.Cu") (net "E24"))
 (segment (start 31.5 44.8) (end 32.799999 44.8) (width 0.1) (layer "B.Cu") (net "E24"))
 (segment (start 26.5 42.4) (end 31.5 44.8) (width 0.1) (layer "B.Cu") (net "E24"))
 (segment (start 31.5 45.4) (end 32 45.4) (width 0.1) (layer "F.Cu") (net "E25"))
 (segment (start 25.6375 42.7) (end 26.5 42.7) (width 0.1) (layer "F.Cu") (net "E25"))
 (segment (start 26.5 42.7) (end 31.5 45.4) (width 0.1) (layer "F.Cu") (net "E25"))
 (via (at 32 45.4) (size 0.55) (drill 0.3) (layers "F.Cu" "B.Cu") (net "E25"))
 (segment (start 38.8 42.7) (end 119.1 42.7) (width 0.1) (layer "B.Cu") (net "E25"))
 (segment (start 32.799999 45.4) (end 38.8 42.7) (width 0.1) (layer "B.Cu") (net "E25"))
 (segment (start 32 45.4) (end 32.799999 45.4) (width 0.1) (layer "B.Cu") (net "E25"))
 (segment (start 22.7625 43) (end 21.7 43) (width 0.1) (layer "F.Cu") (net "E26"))
 (via (at 21.7 43) (size 0.55) (drill 0.3) (layers "F.Cu" "B.Cu") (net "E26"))
 (segment (start 26.5 43) (end 31.5 46) (width 0.1) (layer "B.Cu") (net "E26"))
 (segment (start 32.799999 46) (end 38.8 43) (width 0.1) (layer "B.Cu") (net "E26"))
 (segment (start 21.7 43) (end 26.5 43) (width 0.1) (layer "B.Cu") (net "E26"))
 (segment (start 31.5 46) (end 32.799999 46) (width 0.1) (layer "B.Cu") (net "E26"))
 (segment (start 38.8 43) (end 118 43) (width 0.1) (layer "B.Cu") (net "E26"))
 (segment (start 25.6375 43.3) (end 26.5 43.3) (width 0.1) (layer "F.Cu") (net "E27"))
 (segment (start 31.5 46.6) (end 32 46.6) (width 0.1) (layer "F.Cu") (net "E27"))
 (segment (start 26.5 43.3) (end 31.5 46.6) (width 0.1) (layer "F.Cu") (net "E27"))
 (via (at 32 46.6) (size 0.55) (drill 0.3) (layers "F.Cu" "B.Cu") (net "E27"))
 (segment (start 32.799999 46.6) (end 38.8 43.3) (width 0.1) (layer "B.Cu") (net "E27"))
 (segment (start 38.8 43.3) (end 119.1 43.3) (width 0.1) (layer "B.Cu") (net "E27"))
 (segment (start 32 46.6) (end 32.799999 46.6) (width 0.1) (layer "B.Cu") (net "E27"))
 (segment (start 22.7625 43.6) (end 20.8 43.6) (width 0.1) (layer "F.Cu") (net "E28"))
 (via (at 20.8 43.6) (size 0.55) (drill 0.3) (layers "F.Cu" "B.Cu") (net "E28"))
 (segment (start 31.5 47.2) (end 32.799999 47.2) (width 0.1) (layer "B.Cu") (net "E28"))
 (segment (start 38.8 43.6) (end 118 43.6) (width 0.1) (layer "B.Cu") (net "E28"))
 (segment (start 26.5 43.6) (end 31.5 47.2) (width 0.1) (layer "B.Cu") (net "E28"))
 (segment (start 32.799999 47.2) (end 38.8 43.6) (width 0.1) (layer "B.Cu") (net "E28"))
 (segment (start 20.8 43.6) (end 26.5 43.6) (width 0.1) (layer "B.Cu") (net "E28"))
 (segment (start 25.6375 43.9) (end 26.5 43.9) (width 0.1) (layer "F.Cu") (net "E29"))
 (segment (start 31.5 47.8) (end 32 47.8) (width 0.1) (layer "F.Cu") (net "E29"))
 (segment (start 26.5 43.9) (end 31.5 47.8) (width 0.1) (layer "F.Cu") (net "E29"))
 (via (at 32 47.8) (size 0.55) (drill 0.3) (layers "F.Cu" "B.Cu") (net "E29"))
 (segment (start 32.799999 47.8) (end 38.8 43.9) (width 0.1) (layer "B.Cu") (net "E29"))
 (segment (start 32 47.8) (end 32.799999 47.8) (width 0.1) (layer "B.Cu") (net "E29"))
 (segment (start 38.8 43.9) (end 119.1 43.9) (width 0.1) (layer "B.Cu") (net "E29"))
 (segment (start 22.7625 44.2) (end 21.7 44.2) (width 0.1) (layer "F.Cu") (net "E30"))
 (via (at 21.7 44.2) (size 0.55) (drill 0.3) (layers "F.Cu" "B.Cu") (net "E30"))
 (segment (start 38.8 44.2) (end 118 44.2) (width 0.1) (layer "B.Cu") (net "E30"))
 (segment (start 31.5 48.4) (end 32.799999 48.4) (width 0.1) (layer "B.Cu") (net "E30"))
 (segment (start 21.7 44.2) (end 26.5 44.2) (width 0.1) (layer "B.Cu") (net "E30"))
 (segment (start 32.799999 48.4) (end 38.8 44.2) (width 0.1) (layer "B.Cu") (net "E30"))
 (segment (start 26.5 44.2) (end 31.5 48.4) (width 0.1) (layer "B.Cu") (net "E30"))
 (segment (start 26.5 44.5) (end 31.5 49) (width 0.1) (layer "F.Cu") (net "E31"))
 (segment (start 25.6375 44.5) (end 26.5 44.5) (width 0.1) (layer "F.Cu") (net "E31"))
 (segment (start 31.5 49) (end 32 49) (width 0.1) (layer "F.Cu") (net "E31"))
 (via (at 32 49) (size 0.55) (drill 0.3) (layers "F.Cu" "B.Cu") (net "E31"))
 (segment (start 32.799999 49) (end 38.8 44.5) (width 0.1) (layer "B.Cu") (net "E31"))
 (segment (start 32 49) (end 32.799999 49) (width 0.1) (layer "B.Cu") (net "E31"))
 (segment (start 38.8 44.5) (end 119.1 44.5) (width 0.1) (layer "B.Cu") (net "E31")))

